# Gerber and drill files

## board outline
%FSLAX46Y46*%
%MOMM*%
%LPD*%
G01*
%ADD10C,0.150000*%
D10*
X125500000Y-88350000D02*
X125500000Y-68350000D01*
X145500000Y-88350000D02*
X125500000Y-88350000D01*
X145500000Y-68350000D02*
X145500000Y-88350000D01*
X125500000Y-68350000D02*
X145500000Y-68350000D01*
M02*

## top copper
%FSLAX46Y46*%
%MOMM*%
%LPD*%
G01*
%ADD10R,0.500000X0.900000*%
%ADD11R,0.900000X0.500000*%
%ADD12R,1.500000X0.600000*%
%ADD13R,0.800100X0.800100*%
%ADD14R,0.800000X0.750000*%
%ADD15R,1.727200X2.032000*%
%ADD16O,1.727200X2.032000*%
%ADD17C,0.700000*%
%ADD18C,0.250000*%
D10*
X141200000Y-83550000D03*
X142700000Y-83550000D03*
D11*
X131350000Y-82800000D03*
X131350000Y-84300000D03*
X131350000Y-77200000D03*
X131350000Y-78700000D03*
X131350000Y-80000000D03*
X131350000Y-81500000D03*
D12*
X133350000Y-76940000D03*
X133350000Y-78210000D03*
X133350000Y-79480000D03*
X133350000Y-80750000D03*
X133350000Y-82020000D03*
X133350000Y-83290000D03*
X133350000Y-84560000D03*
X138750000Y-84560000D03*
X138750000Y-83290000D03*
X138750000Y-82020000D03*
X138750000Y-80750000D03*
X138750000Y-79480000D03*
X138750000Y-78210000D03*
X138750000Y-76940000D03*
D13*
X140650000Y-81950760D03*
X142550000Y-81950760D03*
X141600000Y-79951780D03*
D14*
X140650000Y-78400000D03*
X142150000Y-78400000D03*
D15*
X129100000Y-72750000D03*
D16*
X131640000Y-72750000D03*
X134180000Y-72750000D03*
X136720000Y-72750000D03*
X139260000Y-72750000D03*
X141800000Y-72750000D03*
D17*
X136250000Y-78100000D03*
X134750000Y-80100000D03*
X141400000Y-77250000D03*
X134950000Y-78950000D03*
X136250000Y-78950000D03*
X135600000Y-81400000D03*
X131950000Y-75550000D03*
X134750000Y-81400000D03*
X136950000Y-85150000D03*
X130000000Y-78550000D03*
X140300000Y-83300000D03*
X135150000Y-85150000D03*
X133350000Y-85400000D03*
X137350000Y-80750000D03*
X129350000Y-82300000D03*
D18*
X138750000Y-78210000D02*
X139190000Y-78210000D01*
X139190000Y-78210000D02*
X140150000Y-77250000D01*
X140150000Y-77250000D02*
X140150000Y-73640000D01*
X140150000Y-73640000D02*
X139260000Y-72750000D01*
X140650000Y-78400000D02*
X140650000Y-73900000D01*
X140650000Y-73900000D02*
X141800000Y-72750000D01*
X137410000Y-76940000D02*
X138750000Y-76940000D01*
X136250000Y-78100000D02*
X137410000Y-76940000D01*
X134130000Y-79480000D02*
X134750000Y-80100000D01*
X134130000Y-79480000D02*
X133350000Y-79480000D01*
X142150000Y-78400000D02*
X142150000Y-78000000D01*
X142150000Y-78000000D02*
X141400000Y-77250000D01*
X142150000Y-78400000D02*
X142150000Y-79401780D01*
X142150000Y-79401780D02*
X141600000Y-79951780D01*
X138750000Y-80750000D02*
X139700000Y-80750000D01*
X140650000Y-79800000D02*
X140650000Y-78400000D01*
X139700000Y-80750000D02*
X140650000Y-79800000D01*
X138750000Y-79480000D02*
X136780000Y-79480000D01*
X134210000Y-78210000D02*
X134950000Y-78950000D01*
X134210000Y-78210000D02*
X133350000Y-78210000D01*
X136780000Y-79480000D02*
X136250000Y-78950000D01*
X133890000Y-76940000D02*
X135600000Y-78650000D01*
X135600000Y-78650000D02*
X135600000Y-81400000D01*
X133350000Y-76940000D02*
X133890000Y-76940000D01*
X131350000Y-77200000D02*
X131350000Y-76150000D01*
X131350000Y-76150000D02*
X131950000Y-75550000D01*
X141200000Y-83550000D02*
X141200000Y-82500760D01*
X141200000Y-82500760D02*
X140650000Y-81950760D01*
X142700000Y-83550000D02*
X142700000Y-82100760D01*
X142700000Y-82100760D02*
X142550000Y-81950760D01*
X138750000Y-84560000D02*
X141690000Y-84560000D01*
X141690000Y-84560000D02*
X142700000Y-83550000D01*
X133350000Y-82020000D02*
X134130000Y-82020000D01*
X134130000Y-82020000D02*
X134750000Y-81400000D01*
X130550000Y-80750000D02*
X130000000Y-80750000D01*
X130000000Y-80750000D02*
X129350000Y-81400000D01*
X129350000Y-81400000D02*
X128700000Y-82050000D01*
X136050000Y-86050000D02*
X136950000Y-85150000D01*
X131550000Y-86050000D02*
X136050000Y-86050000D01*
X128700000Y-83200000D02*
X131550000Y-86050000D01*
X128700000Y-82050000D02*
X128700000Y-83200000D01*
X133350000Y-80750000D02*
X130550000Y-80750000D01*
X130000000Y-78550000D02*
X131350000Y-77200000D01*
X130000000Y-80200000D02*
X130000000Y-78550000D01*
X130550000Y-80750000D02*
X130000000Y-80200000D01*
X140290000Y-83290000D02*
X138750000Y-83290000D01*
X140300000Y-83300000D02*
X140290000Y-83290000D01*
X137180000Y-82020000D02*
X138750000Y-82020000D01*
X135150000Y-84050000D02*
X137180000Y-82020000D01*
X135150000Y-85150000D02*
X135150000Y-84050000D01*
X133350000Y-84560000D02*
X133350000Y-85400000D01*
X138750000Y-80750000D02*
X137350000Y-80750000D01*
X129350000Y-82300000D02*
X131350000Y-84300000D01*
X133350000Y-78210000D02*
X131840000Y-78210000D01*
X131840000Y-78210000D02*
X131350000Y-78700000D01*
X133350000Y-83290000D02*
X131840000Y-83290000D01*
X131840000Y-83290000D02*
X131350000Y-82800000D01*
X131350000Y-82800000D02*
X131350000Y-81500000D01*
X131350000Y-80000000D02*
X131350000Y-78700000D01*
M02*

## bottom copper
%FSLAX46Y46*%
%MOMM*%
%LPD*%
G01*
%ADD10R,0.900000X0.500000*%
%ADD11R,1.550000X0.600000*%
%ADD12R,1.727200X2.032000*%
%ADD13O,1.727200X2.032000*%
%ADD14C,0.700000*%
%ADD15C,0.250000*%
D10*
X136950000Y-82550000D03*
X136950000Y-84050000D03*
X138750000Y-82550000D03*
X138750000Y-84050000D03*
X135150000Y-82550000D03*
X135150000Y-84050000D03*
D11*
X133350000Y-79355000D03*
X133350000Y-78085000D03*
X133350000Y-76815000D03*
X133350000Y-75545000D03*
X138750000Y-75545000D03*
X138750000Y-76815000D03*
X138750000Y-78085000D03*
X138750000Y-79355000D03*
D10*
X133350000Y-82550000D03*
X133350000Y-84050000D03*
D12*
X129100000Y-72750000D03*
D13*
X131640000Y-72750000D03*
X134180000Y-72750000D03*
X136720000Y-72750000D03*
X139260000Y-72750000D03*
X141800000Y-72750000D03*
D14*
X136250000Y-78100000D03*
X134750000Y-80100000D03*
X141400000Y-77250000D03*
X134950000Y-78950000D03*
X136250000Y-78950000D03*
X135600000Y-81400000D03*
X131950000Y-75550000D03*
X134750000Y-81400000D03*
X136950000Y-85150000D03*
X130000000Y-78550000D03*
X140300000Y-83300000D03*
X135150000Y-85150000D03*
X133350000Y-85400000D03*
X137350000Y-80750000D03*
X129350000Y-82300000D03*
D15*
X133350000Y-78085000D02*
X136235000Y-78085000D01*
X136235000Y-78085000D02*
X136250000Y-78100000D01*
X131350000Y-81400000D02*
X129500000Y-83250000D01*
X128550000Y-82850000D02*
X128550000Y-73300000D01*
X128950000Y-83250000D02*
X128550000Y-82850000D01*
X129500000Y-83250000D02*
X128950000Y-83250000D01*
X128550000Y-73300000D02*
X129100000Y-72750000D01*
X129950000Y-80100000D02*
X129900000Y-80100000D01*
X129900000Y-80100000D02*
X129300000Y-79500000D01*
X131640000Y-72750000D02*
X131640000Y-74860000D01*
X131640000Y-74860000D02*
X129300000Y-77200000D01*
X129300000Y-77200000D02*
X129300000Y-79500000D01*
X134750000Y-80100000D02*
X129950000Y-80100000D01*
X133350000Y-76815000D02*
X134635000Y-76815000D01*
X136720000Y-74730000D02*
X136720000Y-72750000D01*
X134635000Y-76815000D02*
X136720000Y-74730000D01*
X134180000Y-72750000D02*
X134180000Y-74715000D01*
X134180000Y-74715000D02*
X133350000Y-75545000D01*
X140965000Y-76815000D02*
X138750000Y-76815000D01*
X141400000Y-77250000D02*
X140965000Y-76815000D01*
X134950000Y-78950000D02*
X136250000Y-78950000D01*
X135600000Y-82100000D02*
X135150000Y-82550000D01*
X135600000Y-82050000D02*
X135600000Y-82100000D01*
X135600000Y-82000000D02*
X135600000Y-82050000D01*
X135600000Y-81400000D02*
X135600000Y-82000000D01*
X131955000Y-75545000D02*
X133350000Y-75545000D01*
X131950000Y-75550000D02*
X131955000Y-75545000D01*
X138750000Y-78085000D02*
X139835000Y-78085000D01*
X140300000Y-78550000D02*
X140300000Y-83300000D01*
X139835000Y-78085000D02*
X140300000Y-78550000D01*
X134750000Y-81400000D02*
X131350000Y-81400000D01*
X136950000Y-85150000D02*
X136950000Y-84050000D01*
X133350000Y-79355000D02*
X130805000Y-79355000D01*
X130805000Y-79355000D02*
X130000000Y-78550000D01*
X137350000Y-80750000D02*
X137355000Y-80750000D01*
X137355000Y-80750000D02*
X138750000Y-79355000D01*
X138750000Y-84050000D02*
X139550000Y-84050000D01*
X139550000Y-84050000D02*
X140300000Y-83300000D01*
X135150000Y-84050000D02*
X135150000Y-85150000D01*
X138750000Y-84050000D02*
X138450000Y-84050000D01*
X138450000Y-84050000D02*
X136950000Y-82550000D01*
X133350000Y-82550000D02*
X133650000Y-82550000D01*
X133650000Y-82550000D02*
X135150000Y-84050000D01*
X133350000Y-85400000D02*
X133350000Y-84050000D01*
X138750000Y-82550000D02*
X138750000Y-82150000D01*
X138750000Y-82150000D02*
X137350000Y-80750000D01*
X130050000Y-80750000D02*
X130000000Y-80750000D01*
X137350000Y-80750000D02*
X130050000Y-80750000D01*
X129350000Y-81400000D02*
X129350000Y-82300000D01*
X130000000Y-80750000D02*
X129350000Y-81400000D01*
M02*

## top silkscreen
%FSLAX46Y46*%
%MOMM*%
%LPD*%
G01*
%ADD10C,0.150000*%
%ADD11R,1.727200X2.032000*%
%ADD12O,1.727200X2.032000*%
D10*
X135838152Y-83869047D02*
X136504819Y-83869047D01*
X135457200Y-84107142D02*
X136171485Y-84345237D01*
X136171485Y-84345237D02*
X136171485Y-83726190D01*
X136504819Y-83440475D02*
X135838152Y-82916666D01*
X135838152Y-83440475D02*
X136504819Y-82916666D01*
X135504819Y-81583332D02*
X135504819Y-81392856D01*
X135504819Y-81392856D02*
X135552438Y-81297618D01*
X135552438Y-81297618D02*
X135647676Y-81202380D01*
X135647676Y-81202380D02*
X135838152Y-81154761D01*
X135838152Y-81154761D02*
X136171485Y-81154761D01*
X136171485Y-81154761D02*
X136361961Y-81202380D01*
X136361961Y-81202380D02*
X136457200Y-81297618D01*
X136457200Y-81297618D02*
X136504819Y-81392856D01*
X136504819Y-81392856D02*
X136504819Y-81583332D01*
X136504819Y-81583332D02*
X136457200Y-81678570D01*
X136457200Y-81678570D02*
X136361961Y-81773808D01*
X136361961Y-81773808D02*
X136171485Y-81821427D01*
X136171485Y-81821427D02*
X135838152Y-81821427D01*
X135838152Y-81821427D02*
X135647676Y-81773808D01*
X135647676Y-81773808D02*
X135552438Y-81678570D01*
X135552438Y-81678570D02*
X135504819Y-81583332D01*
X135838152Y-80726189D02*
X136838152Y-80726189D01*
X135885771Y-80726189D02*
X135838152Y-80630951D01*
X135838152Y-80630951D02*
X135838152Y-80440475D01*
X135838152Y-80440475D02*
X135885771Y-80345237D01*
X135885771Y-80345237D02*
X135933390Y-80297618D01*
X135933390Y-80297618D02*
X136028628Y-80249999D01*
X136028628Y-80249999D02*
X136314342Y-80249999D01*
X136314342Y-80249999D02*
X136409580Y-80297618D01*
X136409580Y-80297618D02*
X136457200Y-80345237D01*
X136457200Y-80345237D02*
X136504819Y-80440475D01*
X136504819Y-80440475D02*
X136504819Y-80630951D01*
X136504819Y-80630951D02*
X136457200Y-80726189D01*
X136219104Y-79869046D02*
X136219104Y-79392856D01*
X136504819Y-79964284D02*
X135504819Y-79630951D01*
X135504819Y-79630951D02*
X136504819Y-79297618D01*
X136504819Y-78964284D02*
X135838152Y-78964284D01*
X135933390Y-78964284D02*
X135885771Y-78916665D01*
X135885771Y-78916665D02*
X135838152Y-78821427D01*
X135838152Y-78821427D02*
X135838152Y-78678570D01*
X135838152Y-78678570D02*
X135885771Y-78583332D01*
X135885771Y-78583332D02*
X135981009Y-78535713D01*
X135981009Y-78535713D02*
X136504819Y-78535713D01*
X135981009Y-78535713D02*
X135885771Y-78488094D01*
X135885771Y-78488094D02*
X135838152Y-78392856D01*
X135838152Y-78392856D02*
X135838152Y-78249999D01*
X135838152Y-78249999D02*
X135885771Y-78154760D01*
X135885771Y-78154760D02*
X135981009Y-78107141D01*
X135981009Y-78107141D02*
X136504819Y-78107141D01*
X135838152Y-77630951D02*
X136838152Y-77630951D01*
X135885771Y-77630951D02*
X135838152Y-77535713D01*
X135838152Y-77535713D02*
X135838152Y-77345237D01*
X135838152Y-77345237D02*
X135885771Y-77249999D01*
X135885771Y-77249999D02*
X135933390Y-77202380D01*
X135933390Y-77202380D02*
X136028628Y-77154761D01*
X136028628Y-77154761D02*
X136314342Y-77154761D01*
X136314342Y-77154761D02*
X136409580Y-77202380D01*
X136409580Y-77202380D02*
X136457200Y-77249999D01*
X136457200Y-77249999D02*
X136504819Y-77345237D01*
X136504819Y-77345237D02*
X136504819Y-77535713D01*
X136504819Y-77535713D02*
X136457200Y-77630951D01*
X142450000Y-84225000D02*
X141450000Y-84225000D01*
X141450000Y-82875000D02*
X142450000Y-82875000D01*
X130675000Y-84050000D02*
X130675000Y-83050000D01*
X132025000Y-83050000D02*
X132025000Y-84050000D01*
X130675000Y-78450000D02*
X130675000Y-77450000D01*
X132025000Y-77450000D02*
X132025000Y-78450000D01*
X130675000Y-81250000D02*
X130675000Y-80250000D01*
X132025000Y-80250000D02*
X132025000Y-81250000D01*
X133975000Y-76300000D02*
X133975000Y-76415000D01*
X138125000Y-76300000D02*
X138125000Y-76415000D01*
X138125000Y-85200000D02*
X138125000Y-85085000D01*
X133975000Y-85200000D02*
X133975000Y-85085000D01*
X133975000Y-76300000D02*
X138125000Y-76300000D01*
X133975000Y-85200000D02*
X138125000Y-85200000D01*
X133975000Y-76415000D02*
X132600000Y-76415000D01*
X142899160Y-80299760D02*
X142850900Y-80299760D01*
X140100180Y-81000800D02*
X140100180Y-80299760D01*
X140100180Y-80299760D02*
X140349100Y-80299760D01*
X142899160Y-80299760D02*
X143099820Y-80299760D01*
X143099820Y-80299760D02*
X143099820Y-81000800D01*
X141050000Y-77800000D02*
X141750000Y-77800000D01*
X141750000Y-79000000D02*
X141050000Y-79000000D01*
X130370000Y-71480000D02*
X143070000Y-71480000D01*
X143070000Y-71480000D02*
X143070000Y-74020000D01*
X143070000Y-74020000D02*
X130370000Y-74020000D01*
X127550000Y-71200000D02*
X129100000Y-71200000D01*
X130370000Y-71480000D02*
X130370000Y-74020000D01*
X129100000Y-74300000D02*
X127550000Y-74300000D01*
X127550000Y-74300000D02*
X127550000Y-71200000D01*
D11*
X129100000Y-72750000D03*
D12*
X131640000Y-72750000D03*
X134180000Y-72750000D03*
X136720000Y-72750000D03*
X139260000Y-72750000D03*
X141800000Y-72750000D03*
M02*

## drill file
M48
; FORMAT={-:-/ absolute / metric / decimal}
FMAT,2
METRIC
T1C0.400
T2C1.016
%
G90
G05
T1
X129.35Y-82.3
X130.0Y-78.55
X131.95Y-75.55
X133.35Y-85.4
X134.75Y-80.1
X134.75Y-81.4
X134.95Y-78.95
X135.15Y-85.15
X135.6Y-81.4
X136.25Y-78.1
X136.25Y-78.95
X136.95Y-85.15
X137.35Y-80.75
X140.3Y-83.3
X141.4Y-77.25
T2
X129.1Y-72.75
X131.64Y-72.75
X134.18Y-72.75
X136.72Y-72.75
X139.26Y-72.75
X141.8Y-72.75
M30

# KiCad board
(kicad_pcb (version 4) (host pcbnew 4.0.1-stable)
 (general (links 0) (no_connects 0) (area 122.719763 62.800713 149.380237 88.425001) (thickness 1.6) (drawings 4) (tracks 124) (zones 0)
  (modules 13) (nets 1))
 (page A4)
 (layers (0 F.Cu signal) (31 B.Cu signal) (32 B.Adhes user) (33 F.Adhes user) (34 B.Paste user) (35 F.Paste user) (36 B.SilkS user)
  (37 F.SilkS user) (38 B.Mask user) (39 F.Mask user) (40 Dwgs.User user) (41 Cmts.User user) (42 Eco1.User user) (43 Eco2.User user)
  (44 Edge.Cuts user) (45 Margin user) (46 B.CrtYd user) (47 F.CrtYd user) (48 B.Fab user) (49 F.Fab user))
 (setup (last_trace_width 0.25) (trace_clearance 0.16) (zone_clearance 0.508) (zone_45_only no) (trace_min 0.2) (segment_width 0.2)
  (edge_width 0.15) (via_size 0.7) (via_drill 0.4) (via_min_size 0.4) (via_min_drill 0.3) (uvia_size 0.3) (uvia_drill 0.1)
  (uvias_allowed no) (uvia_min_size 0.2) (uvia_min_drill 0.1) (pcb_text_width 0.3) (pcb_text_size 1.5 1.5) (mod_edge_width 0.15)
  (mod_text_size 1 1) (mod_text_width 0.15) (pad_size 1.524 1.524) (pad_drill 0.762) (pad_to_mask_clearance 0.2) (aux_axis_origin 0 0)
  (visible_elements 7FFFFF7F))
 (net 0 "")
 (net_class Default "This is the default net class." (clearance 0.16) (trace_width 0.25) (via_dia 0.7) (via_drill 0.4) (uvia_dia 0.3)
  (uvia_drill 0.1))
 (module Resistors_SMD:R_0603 (layer B.Cu) (at 136.95 83.3 270)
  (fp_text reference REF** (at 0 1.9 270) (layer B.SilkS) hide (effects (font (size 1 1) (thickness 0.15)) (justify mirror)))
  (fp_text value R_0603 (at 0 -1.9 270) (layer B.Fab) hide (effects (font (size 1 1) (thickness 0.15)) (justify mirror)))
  (pad 1 smd rect (at -0.75 0 270) (size 0.5 0.9) (layers B.Cu B.Paste B.Mask))
  (pad 2 smd rect (at 0.75 0 270) (size 0.5 0.9) (layers B.Cu B.Paste B.Mask)))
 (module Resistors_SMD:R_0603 (layer B.Cu) (at 138.75 83.3 270)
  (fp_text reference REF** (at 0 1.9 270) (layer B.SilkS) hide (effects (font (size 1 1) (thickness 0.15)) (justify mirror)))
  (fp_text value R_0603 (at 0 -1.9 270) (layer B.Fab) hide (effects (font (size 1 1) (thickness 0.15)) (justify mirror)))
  (pad 1 smd rect (at -0.75 0 270) (size 0.5 0.9) (layers B.Cu B.Paste B.Mask))
  (pad 2 smd rect (at 0.75 0 270) (size 0.5 0.9) (layers B.Cu B.Paste B.Mask)))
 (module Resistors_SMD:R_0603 (layer F.Cu) (at 141.95 83.55)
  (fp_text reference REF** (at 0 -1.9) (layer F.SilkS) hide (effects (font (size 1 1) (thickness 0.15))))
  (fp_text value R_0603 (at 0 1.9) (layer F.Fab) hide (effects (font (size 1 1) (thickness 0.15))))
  (fp_line (start 0.5 0.675) (end -0.5 0.675) (layer F.SilkS) (width 0.15))
  (fp_line (start -0.5 -0.675) (end 0.5 -0.675) (layer F.SilkS) (width 0.15))
  (pad 1 smd rect (at -0.75 0) (size 0.5 0.9) (layers F.Cu F.Paste F.Mask))
  (pad 2 smd rect (at 0.75 0) (size 0.5 0.9) (layers F.Cu F.Paste F.Mask)))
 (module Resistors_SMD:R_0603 (layer B.Cu) (at 135.15 83.3 270)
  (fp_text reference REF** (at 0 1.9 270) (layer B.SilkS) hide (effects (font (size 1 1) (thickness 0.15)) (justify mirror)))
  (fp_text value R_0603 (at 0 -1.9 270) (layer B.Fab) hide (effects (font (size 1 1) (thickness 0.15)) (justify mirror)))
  (pad 1 smd rect (at -0.75 0 270) (size 0.5 0.9) (layers B.Cu B.Paste B.Mask))
  (pad 2 smd rect (at 0.75 0 270) (size 0.5 0.9) (layers B.Cu B.Paste B.Mask)))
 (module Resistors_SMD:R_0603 (layer F.Cu) (at 131.35 83.55 270)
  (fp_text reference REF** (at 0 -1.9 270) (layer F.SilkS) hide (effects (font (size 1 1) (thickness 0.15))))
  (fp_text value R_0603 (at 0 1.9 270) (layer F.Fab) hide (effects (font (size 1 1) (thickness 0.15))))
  (fp_line (start 0.5 0.675) (end -0.5 0.675) (layer F.SilkS) (width 0.15))
  (fp_line (start -0.5 -0.675) (end 0.5 -0.675) (layer F.SilkS) (width 0.15))
  (pad 1 smd rect (at -0.75 0 270) (size 0.5 0.9) (layers F.Cu F.Paste F.Mask))
  (pad 2 smd rect (at 0.75 0 270) (size 0.5 0.9) (layers F.Cu F.Paste F.Mask)))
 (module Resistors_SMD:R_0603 (layer F.Cu) (at 131.35 77.95 270)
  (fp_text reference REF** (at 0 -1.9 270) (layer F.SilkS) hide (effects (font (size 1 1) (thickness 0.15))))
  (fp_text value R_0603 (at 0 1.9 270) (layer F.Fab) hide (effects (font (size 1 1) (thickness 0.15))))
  (fp_line (start 0.5 0.675) (end -0.5 0.675) (layer F.SilkS) (width 0.15))
  (fp_line (start -0.5 -0.675) (end 0.5 -0.675) (layer F.SilkS) (width 0.15))
  (pad 1 smd rect (at -0.75 0 270) (size 0.5 0.9) (layers F.Cu F.Paste F.Mask))
  (pad 2 smd rect (at 0.75 0 270) (size 0.5 0.9) (layers F.Cu F.Paste F.Mask)))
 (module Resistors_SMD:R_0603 (layer F.Cu) (at 131.35 80.75 270)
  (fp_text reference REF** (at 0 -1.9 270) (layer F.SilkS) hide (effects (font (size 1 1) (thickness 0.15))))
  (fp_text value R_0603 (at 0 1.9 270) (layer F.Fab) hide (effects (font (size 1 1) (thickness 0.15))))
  (fp_line (start 0.5 0.675) (end -0.5 0.675) (layer F.SilkS) (width 0.15))
  (fp_line (start -0.5 -0.675) (end 0.5 -0.675) (layer F.SilkS) (width 0.15))
  (pad 1 smd rect (at -0.75 0 270) (size 0.5 0.9) (layers F.Cu F.Paste F.Mask))
  (pad 2 smd rect (at 0.75 0 270) (size 0.5 0.9) (layers F.Cu F.Paste F.Mask)))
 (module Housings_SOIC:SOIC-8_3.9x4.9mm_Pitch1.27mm (layer B.Cu) (at 136.05 77.45)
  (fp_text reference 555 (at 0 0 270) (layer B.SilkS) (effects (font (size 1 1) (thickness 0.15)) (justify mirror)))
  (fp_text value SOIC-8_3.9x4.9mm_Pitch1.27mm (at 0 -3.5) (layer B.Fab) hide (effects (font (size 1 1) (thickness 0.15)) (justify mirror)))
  (pad 1 smd rect (at -2.7 1.905) (size 1.55 0.6) (layers B.Cu B.Paste B.Mask))
  (pad 2 smd rect (at -2.7 0.635) (size 1.55 0.6) (layers B.Cu B.Paste B.Mask))
  (pad 3 smd rect (at -2.7 -0.635) (size 1.55 0.6) (layers B.Cu B.Paste B.Mask))
  (pad 4 smd rect (at -2.7 -1.905) (size 1.55 0.6) (layers B.Cu B.Paste B.Mask))
  (pad 5 smd rect (at 2.7 -1.905) (size 1.55 0.6) (layers B.Cu B.Paste B.Mask))
  (pad 6 smd rect (at 2.7 -0.635) (size 1.55 0.6) (layers B.Cu B.Paste B.Mask))
  (pad 7 smd rect (at 2.7 0.635) (size 1.55 0.6) (layers B.Cu B.Paste B.Mask))
  (pad 8 smd rect (at 2.7 1.905) (size 1.55 0.6) (layers B.Cu B.Paste B.Mask)))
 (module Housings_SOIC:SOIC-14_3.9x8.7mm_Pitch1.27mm (layer F.Cu) (at 136.05 80.75)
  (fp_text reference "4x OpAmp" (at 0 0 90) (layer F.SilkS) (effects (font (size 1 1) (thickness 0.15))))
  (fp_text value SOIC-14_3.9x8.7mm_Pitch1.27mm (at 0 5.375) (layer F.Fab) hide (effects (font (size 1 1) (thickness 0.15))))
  (fp_line (start -2.075 -4.45) (end -2.075 -4.335) (layer F.SilkS) (width 0.15))
  (fp_line (start 2.075 -4.45) (end 2.075 -4.335) (layer F.SilkS) (width 0.15))
  (fp_line (start 2.075 4.45) (end 2.075 4.335) (layer F.SilkS) (width 0.15))
  (fp_line (start -2.075 4.45) (end -2.075 4.335) (layer F.SilkS) (width 0.15))
  (fp_line (start -2.075 -4.45) (end 2.075 -4.45) (layer F.SilkS) (width 0.15))
  (fp_line (start -2.075 4.45) (end 2.075 4.45) (layer F.SilkS) (width 0.15))
  (fp_line (start -2.075 -4.335) (end -3.45 -4.335) (layer F.SilkS) (width 0.15))
  (pad 1 smd rect (at -2.7 -3.81) (size 1.5 0.6) (layers F.Cu F.Paste F.Mask))
  (pad 2 smd rect (at -2.7 -2.54) (size 1.5 0.6) (layers F.Cu F.Paste F.Mask))
  (pad 3 smd rect (at -2.7 -1.27) (size 1.5 0.6) (layers F.Cu F.Paste F.Mask))
  (pad 4 smd rect (at -2.7 0) (size 1.5 0.6) (layers F.Cu F.Paste F.Mask))
  (pad 5 smd rect (at -2.7 1.27) (size 1.5 0.6) (layers F.Cu F.Paste F.Mask))
  (pad 6 smd rect (at -2.7 2.54) (size 1.5 0.6) (layers F.Cu F.Paste F.Mask))
  (pad 7 smd rect (at -2.7 3.81) (size 1.5 0.6) (layers F.Cu F.Paste F.Mask))
  (pad 8 smd rect (at 2.7 3.81) (size 1.5 0.6) (layers F.Cu F.Paste F.Mask))
  (pad 9 smd rect (at 2.7 2.54) (size 1.5 0.6) (layers F.Cu F.Paste F.Mask))
  (pad 10 smd rect (at 2.7 1.27) (size 1.5 0.6) (layers F.Cu F.Paste F.Mask))
  (pad 11 smd rect (at 2.7 0) (size 1.5 0.6) (layers F.Cu F.Paste F.Mask))
  (pad 12 smd rect (at 2.7 -1.27) (size 1.5 0.6) (layers F.Cu F.Paste F.Mask))
  (pad 13 smd rect (at 2.7 -2.54) (size 1.5 0.6) (layers F.Cu F.Paste F.Mask))
  (pad 14 smd rect (at 2.7 -3.81) (size 1.5 0.6) (layers F.Cu F.Paste F.Mask)))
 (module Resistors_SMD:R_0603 (layer B.Cu) (at 133.35 83.3 270)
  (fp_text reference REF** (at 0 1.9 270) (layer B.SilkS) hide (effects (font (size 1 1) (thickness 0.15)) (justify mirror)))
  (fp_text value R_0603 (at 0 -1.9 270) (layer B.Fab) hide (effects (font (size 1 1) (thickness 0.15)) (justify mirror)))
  (pad 1 smd rect (at -0.75 0 270) (size 0.5 0.9) (layers B.Cu B.Paste B.Mask))
  (pad 2 smd rect (at 0.75 0 270) (size 0.5 0.9) (layers B.Cu B.Paste B.Mask)))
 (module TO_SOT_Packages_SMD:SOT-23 (layer F.Cu) (at 141.6 80.95)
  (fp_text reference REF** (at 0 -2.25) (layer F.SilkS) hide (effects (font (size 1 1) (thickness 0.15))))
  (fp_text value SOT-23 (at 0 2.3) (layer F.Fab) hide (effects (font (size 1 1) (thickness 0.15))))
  (fp_line (start 1.29916 -0.65024) (end 1.2509 -0.65024) (layer F.SilkS) (width 0.15))
  (fp_line (start -1.49982 0.0508) (end -1.49982 -0.65024) (layer F.SilkS) (width 0.15))
  (fp_line (start -1.49982 -0.65024) (end -1.2509 -0.65024) (layer F.SilkS) (width 0.15))
  (fp_line (start 1.29916 -0.65024) (end 1.49982 -0.65024) (layer F.SilkS) (width 0.15))
  (fp_line (start 1.49982 -0.65024) (end 1.49982 0.0508) (layer F.SilkS) (width 0.15))
  (pad 1 smd rect (at -0.95 1.00076) (size 0.8001 0.8001) (layers F.Cu F.Paste F.Mask))
  (pad 2 smd rect (at 0.95 1.00076) (size 0.8001 0.8001) (layers F.Cu F.Paste F.Mask))
  (pad 3 smd rect (at 0 -0.99822) (size 0.8001 0.8001) (layers F.Cu F.Paste F.Mask)))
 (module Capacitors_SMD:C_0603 (layer F.Cu) (at 141.4 78.4)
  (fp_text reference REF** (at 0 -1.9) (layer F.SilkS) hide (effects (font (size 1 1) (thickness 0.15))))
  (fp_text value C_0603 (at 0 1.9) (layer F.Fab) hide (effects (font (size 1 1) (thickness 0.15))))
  (fp_line (start -0.35 -0.6) (end 0.35 -0.6) (layer F.SilkS) (width 0.15))
  (fp_line (start 0.35 0.6) (end -0.35 0.6) (layer F.SilkS) (width 0.15))
  (pad 1 smd rect (at -0.75 0) (size 0.8 0.75) (layers F.Cu F.Paste F.Mask))
  (pad 2 smd rect (at 0.75 0) (size 0.8 0.75) (layers F.Cu F.Paste F.Mask)))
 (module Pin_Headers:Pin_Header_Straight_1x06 (layer F.Cu) (at 129.1 72.75 90)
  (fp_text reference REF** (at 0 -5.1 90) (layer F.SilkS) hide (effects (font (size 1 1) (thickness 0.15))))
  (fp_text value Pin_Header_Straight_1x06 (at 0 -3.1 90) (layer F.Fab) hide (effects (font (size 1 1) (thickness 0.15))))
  (fp_line (start 1.27 1.27) (end 1.27 13.97) (layer F.SilkS) (width 0.15))
  (fp_line (start 1.27 13.97) (end -1.27 13.97) (layer F.SilkS) (width 0.15))
  (fp_line (start -1.27 13.97) (end -1.27 1.27) (layer F.SilkS) (width 0.15))
  (fp_line (start 1.55 -1.55) (end 1.55 0) (layer F.SilkS) (width 0.15))
  (fp_line (start 1.27 1.27) (end -1.27 1.27) (layer F.SilkS) (width 0.15))
  (fp_line (start -1.55 0) (end -1.55 -1.55) (layer F.SilkS) (width 0.15))
  (fp_line (start -1.55 -1.55) (end 1.55 -1.55) (layer F.SilkS) (width 0.15))
  (pad 1 thru_hole rect (at 0 0 90) (size 2.032 1.7272) (drill 1.016) (layers *.Cu *.Mask F.SilkS))
  (pad 2 thru_hole oval (at 0 2.54 90) (size 2.032 1.7272) (drill 1.016) (layers *.Cu *.Mask F.SilkS))
  (pad 3 thru_hole oval (at 0 5.08 90) (size 2.032 1.7272) (drill 1.016) (layers *.Cu *.Mask F.SilkS))
  (pad 4 thru_hole oval (at 0 7.62 90) (size 2.032 1.7272) (drill 1.016) (layers *.Cu *.Mask F.SilkS))
  (pad 5 thru_hole oval (at 0 10.16 90) (size 2.032 1.7272) (drill 1.016) (layers *.Cu *.Mask F.SilkS))
  (pad 6 thru_hole oval (at 0 12.7 90) (size 2.032 1.7272) (drill 1.016) (layers *.Cu *.Mask F.SilkS)))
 (gr_line (start 125.5 88.35) (end 125.5 68.35) (angle 90) (layer Edge.Cuts) (width 0.15))
 (gr_line (start 145.5 88.35) (end 125.5 88.35) (angle 90) (layer Edge.Cuts) (width 0.15))
 (gr_line (start 145.5 68.35) (end 145.5 88.35) (angle 90) (layer Edge.Cuts) (width 0.15))
 (gr_line (start 125.5 68.35) (end 145.5 68.35) (angle 90) (layer Edge.Cuts) (width 0.15))
 (segment (start 138.75 78.21) (end 139.19 78.21) (width 0.25) (layer F.Cu) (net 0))
 (segment (start 139.19 78.21) (end 140.15 77.25) (width 0.25) (layer F.Cu) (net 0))
 (segment (start 140.15 77.25) (end 140.15 73.64) (width 0.25) (layer F.Cu) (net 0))
 (segment (start 140.15 73.64) (end 139.26 72.75) (width 0.25) (layer F.Cu) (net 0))
 (segment (start 140.65 78.4) (end 140.65 73.9) (width 0.25) (layer F.Cu) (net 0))
 (segment (start 140.65 73.9) (end 141.8 72.75) (width 0.25) (layer F.Cu) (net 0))
 (segment (start 133.35 78.085) (end 136.235 78.085) (width 0.25) (layer B.Cu) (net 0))
 (segment (start 137.41 76.94) (end 138.75 76.94) (width 0.25) (layer F.Cu) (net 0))
 (segment (start 136.25 78.1) (end 137.41 76.94) (width 0.25) (layer F.Cu) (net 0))
 (via (at 136.25 78.1) (size 0.7) (drill 0.4) (layers F.Cu B.Cu) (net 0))
 (segment (start 136.235 78.085) (end 136.25 78.1) (width 0.25) (layer B.Cu) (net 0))
 (segment (start 131.35 81.4) (end 129.5 83.25) (width 0.25) (layer B.Cu) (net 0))
 (segment (start 128.55 82.85) (end 128.55 73.3) (width 0.25) (layer B.Cu) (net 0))
 (segment (start 128.95 83.25) (end 128.55 82.85) (width 0.25) (layer B.Cu) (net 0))
 (segment (start 129.5 83.25) (end 128.95 83.25) (width 0.25) (layer B.Cu) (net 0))
 (segment (start 128.55 73.3) (end 129.1 72.75) (width 0.25) (layer B.Cu) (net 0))
 (segment (start 129.95 80.1) (end 129.9 80.1) (width 0.25) (layer B.Cu) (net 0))
 (segment (start 129.9 80.1) (end 129.3 79.5) (width 0.25) (layer B.Cu) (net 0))
 (segment (start 131.64 72.75) (end 131.64 74.86) (width 0.25) (layer B.Cu) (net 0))
 (segment (start 131.64 74.86) (end 129.3 77.2) (width 0.25) (layer B.Cu) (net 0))
 (segment (start 129.3 77.2) (end 129.3 79.5) (width 0.25) (layer B.Cu) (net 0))
 (segment (start 134.13 79.48) (end 134.75 80.1) (width 0.25) (layer F.Cu) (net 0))
 (via (at 134.75 80.1) (size 0.7) (drill 0.4) (layers F.Cu B.Cu) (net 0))
 (segment (start 134.75 80.1) (end 129.95 80.1) (width 0.25) (layer B.Cu) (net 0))
 (segment (start 134.13 79.48) (end 133.35 79.48) (width 0.25) (layer F.Cu) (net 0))
 (segment (start 133.35 76.815) (end 134.635 76.815) (width 0.25) (layer B.Cu) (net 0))
 (segment (start 136.72 74.73) (end 136.72 72.75) (width 0.25) (layer B.Cu) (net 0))
 (segment (start 134.635 76.815) (end 136.72 74.73) (width 0.25) (layer B.Cu) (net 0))
 (segment (start 134.18 72.75) (end 134.18 74.715) (width 0.25) (layer B.Cu) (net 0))
 (segment (start 134.18 74.715) (end 133.35 75.545) (width 0.25) (layer B.Cu) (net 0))
 (segment (start 142.15 78.4) (end 142.15 78) (width 0.25) (layer F.Cu) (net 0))
 (segment (start 140.965 76.815) (end 138.75 76.815) (width 0.25) (layer B.Cu) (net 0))
 (segment (start 141.4 77.25) (end 140.965 76.815) (width 0.25) (layer B.Cu) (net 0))
 (via (at 141.4 77.25) (size 0.7) (drill 0.4) (layers F.Cu B.Cu) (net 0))
 (segment (start 142.15 78) (end 141.4 77.25) (width 0.25) (layer F.Cu) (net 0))
 (segment (start 142.15 78.4) (end 142.15 79.40178) (width 0.25) (layer F.Cu) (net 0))
 (segment (start 142.15 79.40178) (end 141.6 79.95178) (width 0.25) (layer F.Cu) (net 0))
 (segment (start 138.75 80.75) (end 139.7 80.75) (width 0.25) (layer F.Cu) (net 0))
 (segment (start 140.65 79.8) (end 140.65 78.4) (width 0.25) (layer F.Cu) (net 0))
 (segment (start 139.7 80.75) (end 140.65 79.8) (width 0.25) (layer F.Cu) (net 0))
 (segment (start 138.75 79.48) (end 136.78 79.48) (width 0.25) (layer F.Cu) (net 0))
 (segment (start 134.21 78.21) (end 134.95 78.95) (width 0.25) (layer F.Cu) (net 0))
 (via (at 134.95 78.95) (size 0.7) (drill 0.4) (layers F.Cu B.Cu) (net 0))
 (segment (start 134.95 78.95) (end 136.25 78.95) (width 0.25) (layer B.Cu) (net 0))
 (via (at 136.25 78.95) (size 0.7) (drill 0.4) (layers F.Cu B.Cu) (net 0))
 (segment (start 134.21 78.21) (end 133.35 78.21) (width 0.25) (layer F.Cu) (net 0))
 (segment (start 136.78 79.48) (end 136.25 78.95) (width 0.25) (layer F.Cu) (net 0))
 (segment (start 133.89 76.94) (end 135.6 78.65) (width 0.25) (layer F.Cu) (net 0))
 (segment (start 135.6 82.1) (end 135.15 82.55) (width 0.25) (layer B.Cu) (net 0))
 (segment (start 135.6 82.05) (end 135.6 82.1) (width 0.25) (layer B.Cu) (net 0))
 (segment (start 135.6 82) (end 135.6 82.05) (width 0.25) (layer B.Cu) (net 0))
 (segment (start 135.6 81.4) (end 135.6 82) (width 0.25) (layer B.Cu) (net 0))
 (via (at 135.6 81.4) (size 0.7) (drill 0.4) (layers F.Cu B.Cu) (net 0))
 (segment (start 135.6 78.65) (end 135.6 81.4) (width 0.25) (layer F.Cu) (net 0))
 (segment (start 133.35 76.94) (end 133.89 76.94) (width 0.25) (layer F.Cu) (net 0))
 (segment (start 131.35 77.2) (end 131.35 76.15) (width 0.25) (layer F.Cu) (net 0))
 (segment (start 131.955 75.545) (end 133.35 75.545) (width 0.25) (layer B.Cu) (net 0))
 (segment (start 131.95 75.55) (end 131.955 75.545) (width 0.25) (layer B.Cu) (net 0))
 (via (at 131.95 75.55) (size 0.7) (drill 0.4) (layers F.Cu B.Cu) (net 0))
 (segment (start 131.35 76.15) (end 131.95 75.55) (width 0.25) (layer F.Cu) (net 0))
 (segment (start 141.2 83.55) (end 141.2 82.50076) (width 0.25) (layer F.Cu) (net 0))
 (segment (start 141.2 82.50076) (end 140.65 81.95076) (width 0.25) (layer F.Cu) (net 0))
 (segment (start 142.7 83.55) (end 142.7 82.10076) (width 0.25) (layer F.Cu) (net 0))
 (segment (start 142.7 82.10076) (end 142.55 81.95076) (width 0.25) (layer F.Cu) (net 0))
 (segment (start 138.75 84.56) (end 141.69 84.56) (width 0.25) (layer F.Cu) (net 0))
 (segment (start 141.69 84.56) (end 142.7 83.55) (width 0.25) (layer F.Cu) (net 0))
 (segment (start 138.75 78.085) (end 139.835 78.085) (width 0.25) (layer B.Cu) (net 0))
 (segment (start 140.3 78.55) (end 140.3 83.3) (width 0.25) (layer B.Cu) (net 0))
 (segment (start 139.835 78.085) (end 140.3 78.55) (width 0.25) (layer B.Cu) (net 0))
 (segment (start 133.35 82.02) (end 134.13 82.02) (width 0.25) (layer F.Cu) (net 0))
 (segment (start 134.75 81.4) (end 131.35 81.4) (width 0.25) (layer B.Cu) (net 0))
 (via (at 134.75 81.4) (size 0.7) (drill 0.4) (layers F.Cu B.Cu) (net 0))
 (segment (start 134.13 82.02) (end 134.75 81.4) (width 0.25) (layer F.Cu) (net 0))
 (segment (start 130.55 80.75) (end 130 80.75) (width 0.25) (layer F.Cu) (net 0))
 (segment (start 130 80.75) (end 129.35 81.4) (width 0.25) (layer F.Cu) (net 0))
 (segment (start 129.35 81.4) (end 128.7 82.05) (width 0.25) (layer F.Cu) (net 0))
 (segment (start 136.95 85.15) (end 136.95 84.05) (width 0.25) (layer B.Cu) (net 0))
 (via (at 136.95 85.15) (size 0.7) (drill 0.4) (layers F.Cu B.Cu) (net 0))
 (segment (start 136.05 86.05) (end 136.95 85.15) (width 0.25) (layer F.Cu) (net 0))
 (segment (start 131.55 86.05) (end 136.05 86.05) (width 0.25) (layer F.Cu) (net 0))
 (segment (start 128.7 83.2) (end 131.55 86.05) (width 0.25) (layer F.Cu) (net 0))
 (segment (start 128.7 82.05) (end 128.7 83.2) (width 0.25) (layer F.Cu) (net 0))
 (via (at 130 78.55) (size 0.7) (drill 0.4) (layers F.Cu B.Cu) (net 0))
 (segment (start 133.35 79.355) (end 130.805 79.355) (width 0.25) (layer B.Cu) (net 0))
 (segment (start 130.805 79.355) (end 130 78.55) (width 0.25) (layer B.Cu) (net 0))
 (segment (start 133.35 80.75) (end 130.55 80.75) (width 0.25) (layer F.Cu) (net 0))
 (segment (start 130 78.55) (end 131.35 77.2) (width 0.25) (layer F.Cu) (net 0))
 (segment (start 130 80.2) (end 130 78.55) (width 0.25) (layer F.Cu) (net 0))
 (segment (start 130.55 80.75) (end 130 80.2) (width 0.25) (layer F.Cu) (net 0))
 (segment (start 137.35 80.75) (end 137.355 80.75) (width 0.25) (layer B.Cu) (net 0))
 (segment (start 137.355 80.75) (end 138.75 79.355) (width 0.25) (layer B.Cu) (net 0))
 (segment (start 138.75 84.05) (end 139.55 84.05) (width 0.25) (layer B.Cu) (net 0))
 (segment (start 140.29 83.29) (end 138.75 83.29) (width 0.25) (layer F.Cu) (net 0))
 (segment (start 140.3 83.3) (end 140.29 83.29) (width 0.25) (layer F.Cu) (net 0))
 (via (at 140.3 83.3) (size 0.7) (drill 0.4) (layers F.Cu B.Cu) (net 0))
 (segment (start 139.55 84.05) (end 140.3 83.3) (width 0.25) (layer B.Cu) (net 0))
 (segment (start 135.15 84.05) (end 135.15 85.15) (width 0.25) (layer B.Cu) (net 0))
 (segment (start 137.18 82.02) (end 138.75 82.02) (width 0.25) (layer F.Cu) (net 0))
 (segment (start 135.15 84.05) (end 137.18 82.02) (width 0.25) (layer F.Cu) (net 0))
 (segment (start 135.15 85.15) (end 135.15 84.05) (width 0.25) (layer F.Cu) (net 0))
 (via (at 135.15 85.15) (size 0.7) (drill 0.4) (layers F.Cu B.Cu) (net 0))
 (segment (start 138.75 84.05) (end 138.45 84.05) (width 0.25) (layer B.Cu) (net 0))
 (segment (start 138.45 84.05) (end 136.95 82.55) (width 0.25) (layer B.Cu) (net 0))
 (segment (start 133.35 82.55) (end 133.65 82.55) (width 0.25) (layer B.Cu) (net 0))
 (segment (start 133.65 82.55) (end 135.15 84.05) (width 0.25) (layer B.Cu) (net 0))
 (segment (start 133.35 84.56) (end 133.35 85.4) (width 0.25) (layer F.Cu) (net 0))
 (segment (start 133.35 85.4) (end 133.35 84.05) (width 0.25) (layer B.Cu) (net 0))
 (via (at 133.35 85.4) (size 0.7) (drill 0.4) (layers F.Cu B.Cu) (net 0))
 (segment (start 138.75 82.55) (end 138.75 82.15) (width 0.25) (layer B.Cu) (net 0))
 (segment (start 138.75 82.15) (end 137.35 80.75) (width 0.25) (layer B.Cu) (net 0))
 (segment (start 130.05 80.75) (end 130 80.75) (width 0.25) (layer B.Cu) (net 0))
 (via (at 137.35 80.75) (size 0.7) (drill 0.4) (layers F.Cu B.Cu) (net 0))
 (segment (start 137.35 80.75) (end 130.05 80.75) (width 0.25) (layer B.Cu) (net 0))
 (segment (start 138.75 80.75) (end 137.35 80.75) (width 0.25) (layer F.Cu) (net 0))
 (segment (start 129.35 82.3) (end 131.35 84.3) (width 0.25) (layer F.Cu) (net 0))
 (via (at 129.35 82.3) (size 0.7) (drill 0.4) (layers F.Cu B.Cu) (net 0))
 (segment (start 129.35 81.4) (end 129.35 82.3) (width 0.25) (layer B.Cu) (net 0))
 (segment (start 130 80.75) (end 129.35 81.4) (width 0.25) (layer B.Cu) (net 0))
 (segment (start 133.35 78.21) (end 131.84 78.21) (width 0.25) (layer F.Cu) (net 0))
 (segment (start 131.84 78.21) (end 131.35 78.7) (width 0.25) (layer F.Cu) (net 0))
 (segment (start 133.35 83.29) (end 131.84 83.29) (width 0.25) (layer F.Cu) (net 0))
 (segment (start 131.84 83.29) (end 131.35 82.8) (width 0.25) (layer F.Cu) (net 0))
 (segment (start 131.35 82.8) (end 131.35 81.5) (width 0.25) (layer F.Cu) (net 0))
 (segment (start 131.35 80) (end 131.35 78.7) (width 0.25) (layer F.Cu) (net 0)))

